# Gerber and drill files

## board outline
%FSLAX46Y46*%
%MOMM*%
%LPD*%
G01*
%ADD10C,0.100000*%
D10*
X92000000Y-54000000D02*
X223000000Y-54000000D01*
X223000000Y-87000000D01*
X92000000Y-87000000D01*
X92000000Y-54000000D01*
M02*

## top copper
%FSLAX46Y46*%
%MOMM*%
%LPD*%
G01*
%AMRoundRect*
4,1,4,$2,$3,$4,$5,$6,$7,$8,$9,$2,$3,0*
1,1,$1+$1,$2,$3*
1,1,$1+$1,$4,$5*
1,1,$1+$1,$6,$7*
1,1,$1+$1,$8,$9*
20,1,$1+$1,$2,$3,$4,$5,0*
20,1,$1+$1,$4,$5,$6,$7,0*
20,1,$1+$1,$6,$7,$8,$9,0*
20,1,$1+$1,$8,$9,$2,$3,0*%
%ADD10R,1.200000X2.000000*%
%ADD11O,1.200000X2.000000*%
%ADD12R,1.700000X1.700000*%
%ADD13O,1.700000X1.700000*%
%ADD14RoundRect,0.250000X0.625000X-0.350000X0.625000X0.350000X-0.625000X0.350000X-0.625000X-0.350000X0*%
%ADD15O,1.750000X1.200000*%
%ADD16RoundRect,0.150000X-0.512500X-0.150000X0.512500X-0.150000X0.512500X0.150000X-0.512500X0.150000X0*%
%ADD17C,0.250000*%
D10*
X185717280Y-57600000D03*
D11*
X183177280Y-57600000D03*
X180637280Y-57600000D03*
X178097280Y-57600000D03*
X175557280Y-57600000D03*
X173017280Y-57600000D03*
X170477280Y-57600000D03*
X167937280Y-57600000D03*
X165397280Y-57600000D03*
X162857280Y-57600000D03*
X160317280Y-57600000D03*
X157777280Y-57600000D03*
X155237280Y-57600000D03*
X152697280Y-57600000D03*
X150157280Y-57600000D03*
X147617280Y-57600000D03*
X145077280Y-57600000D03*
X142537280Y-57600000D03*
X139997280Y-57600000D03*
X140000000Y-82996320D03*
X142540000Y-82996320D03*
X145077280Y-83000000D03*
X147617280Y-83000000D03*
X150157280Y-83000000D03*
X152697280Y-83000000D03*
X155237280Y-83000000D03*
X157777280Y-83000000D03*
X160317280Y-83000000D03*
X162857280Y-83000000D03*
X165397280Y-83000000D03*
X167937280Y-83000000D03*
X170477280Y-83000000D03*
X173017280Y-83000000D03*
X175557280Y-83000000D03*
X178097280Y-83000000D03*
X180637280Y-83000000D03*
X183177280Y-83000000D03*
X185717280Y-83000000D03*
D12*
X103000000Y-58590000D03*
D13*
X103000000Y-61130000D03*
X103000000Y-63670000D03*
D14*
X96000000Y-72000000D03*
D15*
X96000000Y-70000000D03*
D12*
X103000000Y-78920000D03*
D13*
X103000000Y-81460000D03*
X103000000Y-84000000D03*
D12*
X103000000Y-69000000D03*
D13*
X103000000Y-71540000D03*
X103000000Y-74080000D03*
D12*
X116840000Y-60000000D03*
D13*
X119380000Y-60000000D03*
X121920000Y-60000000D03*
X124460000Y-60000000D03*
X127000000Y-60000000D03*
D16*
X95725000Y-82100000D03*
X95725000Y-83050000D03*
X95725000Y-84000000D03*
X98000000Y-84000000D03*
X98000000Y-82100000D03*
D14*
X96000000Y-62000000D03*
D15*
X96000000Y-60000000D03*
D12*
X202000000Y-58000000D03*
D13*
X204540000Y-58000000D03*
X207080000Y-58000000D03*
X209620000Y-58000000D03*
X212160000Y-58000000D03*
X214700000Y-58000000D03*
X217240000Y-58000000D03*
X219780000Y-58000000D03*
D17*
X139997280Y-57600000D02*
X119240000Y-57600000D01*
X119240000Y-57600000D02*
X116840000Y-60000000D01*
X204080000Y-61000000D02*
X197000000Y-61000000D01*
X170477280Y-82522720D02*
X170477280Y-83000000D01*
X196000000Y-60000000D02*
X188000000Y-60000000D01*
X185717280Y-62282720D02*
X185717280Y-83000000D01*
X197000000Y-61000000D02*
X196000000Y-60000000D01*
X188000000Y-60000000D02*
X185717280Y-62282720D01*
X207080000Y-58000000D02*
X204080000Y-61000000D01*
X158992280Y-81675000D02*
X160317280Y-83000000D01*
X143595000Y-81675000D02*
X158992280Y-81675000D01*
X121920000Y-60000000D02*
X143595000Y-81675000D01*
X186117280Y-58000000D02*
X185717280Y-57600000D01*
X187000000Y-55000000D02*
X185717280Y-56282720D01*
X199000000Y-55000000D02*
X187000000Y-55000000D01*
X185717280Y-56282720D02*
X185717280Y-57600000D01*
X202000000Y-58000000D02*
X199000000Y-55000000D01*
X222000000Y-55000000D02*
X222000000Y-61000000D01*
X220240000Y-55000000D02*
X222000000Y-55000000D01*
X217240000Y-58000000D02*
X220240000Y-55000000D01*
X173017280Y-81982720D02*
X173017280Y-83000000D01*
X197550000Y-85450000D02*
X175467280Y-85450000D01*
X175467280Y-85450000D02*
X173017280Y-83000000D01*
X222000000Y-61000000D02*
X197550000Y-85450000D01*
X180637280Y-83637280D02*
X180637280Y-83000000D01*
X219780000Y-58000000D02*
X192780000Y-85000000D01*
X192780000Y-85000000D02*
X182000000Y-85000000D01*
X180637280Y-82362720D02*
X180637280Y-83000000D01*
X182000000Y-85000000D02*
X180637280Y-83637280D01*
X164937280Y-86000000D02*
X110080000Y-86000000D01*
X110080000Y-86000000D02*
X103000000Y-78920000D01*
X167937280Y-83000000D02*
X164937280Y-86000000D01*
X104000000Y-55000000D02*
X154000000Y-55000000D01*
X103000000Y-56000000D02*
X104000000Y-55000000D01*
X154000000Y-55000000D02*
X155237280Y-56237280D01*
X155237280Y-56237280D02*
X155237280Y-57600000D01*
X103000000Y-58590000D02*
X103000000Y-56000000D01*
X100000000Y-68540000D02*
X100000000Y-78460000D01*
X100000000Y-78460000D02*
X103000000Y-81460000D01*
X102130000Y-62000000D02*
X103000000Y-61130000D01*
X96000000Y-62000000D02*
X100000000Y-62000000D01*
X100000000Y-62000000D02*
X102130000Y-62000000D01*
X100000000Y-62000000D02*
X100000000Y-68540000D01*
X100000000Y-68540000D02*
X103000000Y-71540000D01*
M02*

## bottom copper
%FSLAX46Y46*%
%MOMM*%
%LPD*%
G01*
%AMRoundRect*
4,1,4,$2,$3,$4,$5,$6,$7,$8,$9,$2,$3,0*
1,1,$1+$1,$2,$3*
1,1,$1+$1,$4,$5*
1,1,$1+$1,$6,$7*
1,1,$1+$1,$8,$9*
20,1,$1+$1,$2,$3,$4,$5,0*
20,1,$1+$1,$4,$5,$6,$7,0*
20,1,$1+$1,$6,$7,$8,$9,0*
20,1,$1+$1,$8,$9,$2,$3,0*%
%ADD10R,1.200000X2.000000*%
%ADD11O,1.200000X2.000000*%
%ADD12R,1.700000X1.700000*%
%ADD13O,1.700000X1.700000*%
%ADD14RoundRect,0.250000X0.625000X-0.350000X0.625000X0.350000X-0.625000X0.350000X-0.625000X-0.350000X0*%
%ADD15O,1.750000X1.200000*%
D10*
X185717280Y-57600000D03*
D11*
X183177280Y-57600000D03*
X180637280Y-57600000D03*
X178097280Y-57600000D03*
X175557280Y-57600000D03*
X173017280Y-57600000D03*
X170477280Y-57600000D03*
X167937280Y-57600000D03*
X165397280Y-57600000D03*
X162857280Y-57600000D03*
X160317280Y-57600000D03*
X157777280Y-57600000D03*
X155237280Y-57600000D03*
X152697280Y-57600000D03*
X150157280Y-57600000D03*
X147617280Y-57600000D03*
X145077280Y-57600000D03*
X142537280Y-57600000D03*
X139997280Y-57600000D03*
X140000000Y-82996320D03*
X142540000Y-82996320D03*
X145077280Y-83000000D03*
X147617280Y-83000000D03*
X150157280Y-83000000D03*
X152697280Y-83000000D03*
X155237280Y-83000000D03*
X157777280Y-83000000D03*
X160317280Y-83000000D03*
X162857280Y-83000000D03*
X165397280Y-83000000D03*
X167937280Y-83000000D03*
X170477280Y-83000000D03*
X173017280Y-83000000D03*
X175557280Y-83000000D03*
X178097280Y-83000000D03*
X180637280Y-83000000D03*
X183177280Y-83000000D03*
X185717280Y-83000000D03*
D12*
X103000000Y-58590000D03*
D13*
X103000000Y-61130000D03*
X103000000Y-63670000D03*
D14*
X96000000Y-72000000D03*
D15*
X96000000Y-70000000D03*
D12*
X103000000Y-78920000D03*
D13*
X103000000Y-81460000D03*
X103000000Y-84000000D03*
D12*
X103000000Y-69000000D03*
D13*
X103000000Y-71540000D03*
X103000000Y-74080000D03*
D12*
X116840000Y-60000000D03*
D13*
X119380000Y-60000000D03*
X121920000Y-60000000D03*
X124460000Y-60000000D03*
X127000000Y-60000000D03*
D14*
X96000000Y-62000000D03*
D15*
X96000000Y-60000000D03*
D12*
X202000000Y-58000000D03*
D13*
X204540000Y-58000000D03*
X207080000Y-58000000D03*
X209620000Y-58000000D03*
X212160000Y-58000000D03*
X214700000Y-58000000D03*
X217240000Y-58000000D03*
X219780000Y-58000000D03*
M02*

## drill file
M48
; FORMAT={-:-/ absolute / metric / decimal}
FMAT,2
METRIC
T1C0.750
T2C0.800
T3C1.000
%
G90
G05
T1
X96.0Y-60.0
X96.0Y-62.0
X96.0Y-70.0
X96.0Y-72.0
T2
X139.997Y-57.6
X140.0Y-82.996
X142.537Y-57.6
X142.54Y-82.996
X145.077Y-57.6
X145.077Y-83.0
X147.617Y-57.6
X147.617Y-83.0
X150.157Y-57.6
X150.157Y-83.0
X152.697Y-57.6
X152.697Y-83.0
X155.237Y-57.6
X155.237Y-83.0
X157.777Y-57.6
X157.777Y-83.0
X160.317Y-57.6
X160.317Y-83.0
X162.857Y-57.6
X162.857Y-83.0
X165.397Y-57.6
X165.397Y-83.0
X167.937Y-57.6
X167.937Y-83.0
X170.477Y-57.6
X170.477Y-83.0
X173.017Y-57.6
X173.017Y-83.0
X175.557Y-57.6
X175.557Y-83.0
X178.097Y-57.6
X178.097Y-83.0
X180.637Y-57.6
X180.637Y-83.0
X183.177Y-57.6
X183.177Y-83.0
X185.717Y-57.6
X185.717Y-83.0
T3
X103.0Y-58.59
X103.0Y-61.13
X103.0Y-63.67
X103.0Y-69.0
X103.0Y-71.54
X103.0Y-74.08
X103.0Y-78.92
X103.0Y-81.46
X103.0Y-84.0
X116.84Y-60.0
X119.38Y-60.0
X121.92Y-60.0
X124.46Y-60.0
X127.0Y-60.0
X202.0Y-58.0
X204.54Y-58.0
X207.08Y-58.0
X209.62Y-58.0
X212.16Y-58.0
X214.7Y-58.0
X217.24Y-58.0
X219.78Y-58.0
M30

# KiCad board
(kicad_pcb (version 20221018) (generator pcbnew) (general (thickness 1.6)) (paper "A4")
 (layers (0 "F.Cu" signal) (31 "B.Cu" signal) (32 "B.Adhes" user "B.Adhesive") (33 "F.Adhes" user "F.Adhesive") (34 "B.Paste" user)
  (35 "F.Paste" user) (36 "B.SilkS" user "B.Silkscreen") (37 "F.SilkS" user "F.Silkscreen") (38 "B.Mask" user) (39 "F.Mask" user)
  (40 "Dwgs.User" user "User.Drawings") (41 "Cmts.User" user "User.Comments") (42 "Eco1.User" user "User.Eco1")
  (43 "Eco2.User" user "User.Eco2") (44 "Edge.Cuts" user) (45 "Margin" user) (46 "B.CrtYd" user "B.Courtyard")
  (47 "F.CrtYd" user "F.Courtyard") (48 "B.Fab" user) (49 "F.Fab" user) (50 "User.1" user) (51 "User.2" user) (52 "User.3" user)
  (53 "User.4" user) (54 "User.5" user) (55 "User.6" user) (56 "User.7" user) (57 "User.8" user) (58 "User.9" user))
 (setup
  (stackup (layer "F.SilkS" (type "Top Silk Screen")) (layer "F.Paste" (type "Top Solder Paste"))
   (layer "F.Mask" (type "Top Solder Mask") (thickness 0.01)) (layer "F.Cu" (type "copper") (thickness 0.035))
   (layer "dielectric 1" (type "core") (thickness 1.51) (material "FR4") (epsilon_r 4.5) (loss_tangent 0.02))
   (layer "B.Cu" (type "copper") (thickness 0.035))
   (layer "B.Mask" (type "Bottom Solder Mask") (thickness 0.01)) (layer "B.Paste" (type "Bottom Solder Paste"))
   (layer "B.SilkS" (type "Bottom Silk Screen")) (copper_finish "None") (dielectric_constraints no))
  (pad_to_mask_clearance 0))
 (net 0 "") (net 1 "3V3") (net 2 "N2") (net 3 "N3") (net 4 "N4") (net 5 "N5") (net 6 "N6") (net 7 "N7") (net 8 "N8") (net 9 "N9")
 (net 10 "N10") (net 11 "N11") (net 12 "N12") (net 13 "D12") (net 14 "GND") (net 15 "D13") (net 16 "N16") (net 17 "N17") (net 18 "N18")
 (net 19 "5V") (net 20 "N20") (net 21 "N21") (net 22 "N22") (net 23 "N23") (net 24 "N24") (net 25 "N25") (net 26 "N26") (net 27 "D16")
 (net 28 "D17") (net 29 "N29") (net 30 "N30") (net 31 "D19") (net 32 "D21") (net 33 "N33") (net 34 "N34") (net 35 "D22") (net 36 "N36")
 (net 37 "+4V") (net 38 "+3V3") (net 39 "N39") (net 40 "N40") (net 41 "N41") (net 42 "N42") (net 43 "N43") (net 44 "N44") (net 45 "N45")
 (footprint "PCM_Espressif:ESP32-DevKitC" (layer "F.Cu") (at 185.71728 57.6 -90)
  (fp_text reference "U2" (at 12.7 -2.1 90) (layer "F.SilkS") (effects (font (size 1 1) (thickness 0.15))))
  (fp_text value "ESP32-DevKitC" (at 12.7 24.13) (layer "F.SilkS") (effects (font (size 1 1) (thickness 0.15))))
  (pad "1" thru_hole rect (at 0 0 180) (size 1.2 2) (drill 0.8) (layers "*.Cu" "*.Mask") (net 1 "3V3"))
  (pad "2" thru_hole oval (at 0 2.54 180) (size 1.2 2) (drill 0.8) (layers "*.Cu" "*.Mask") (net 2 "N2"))
  (pad "3" thru_hole oval (at 0 5.08 180) (size 1.2 2) (drill 0.8) (layers "*.Cu" "*.Mask") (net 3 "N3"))
  (pad "4" thru_hole oval (at 0 7.62 180) (size 1.2 2) (drill 0.8) (layers "*.Cu" "*.Mask") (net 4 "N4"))
  (pad "5" thru_hole oval (at 0 10.16 180) (size 1.2 2) (drill 0.8) (layers "*.Cu" "*.Mask") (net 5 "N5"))
  (pad "6" thru_hole oval (at 0 12.7 180) (size 1.2 2) (drill 0.8) (layers "*.Cu" "*.Mask") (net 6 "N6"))
  (pad "7" thru_hole oval (at 0 15.24 180) (size 1.2 2) (drill 0.8) (layers "*.Cu" "*.Mask") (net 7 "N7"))
  (pad "8" thru_hole oval (at 0 17.78 180) (size 1.2 2) (drill 0.8) (layers "*.Cu" "*.Mask") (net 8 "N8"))
  (pad "9" thru_hole oval (at 0 20.32 180) (size 1.2 2) (drill 0.8) (layers "*.Cu" "*.Mask") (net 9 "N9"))
  (pad "10" thru_hole oval (at 0 22.86 180) (size 1.2 2) (drill 0.8) (layers "*.Cu" "*.Mask") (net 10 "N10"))
  (pad "11" thru_hole oval (at 0 25.4 180) (size 1.2 2) (drill 0.8) (layers "*.Cu" "*.Mask") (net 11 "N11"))
  (pad "12" thru_hole oval (at 0 27.94 180) (size 1.2 2) (drill 0.8) (layers "*.Cu" "*.Mask") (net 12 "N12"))
  (pad "13" thru_hole oval (at 0 30.48 180) (size 1.2 2) (drill 0.8) (layers "*.Cu" "*.Mask") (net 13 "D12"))
  (pad "14" thru_hole oval (at 0 33.02 180) (size 1.2 2) (drill 0.8) (layers "*.Cu" "*.Mask") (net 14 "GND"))
  (pad "15" thru_hole oval (at 0 35.56 180) (size 1.2 2) (drill 0.8) (layers "*.Cu" "*.Mask") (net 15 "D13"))
  (pad "16" thru_hole oval (at 0 38.1 180) (size 1.2 2) (drill 0.8) (layers "*.Cu" "*.Mask") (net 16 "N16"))
  (pad "17" thru_hole oval (at 0 40.64 180) (size 1.2 2) (drill 0.8) (layers "*.Cu" "*.Mask") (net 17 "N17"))
  (pad "18" thru_hole oval (at 0 43.18 180) (size 1.2 2) (drill 0.8) (layers "*.Cu" "*.Mask") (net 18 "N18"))
  (pad "19" thru_hole oval (at 0 45.72 180) (size 1.2 2) (drill 0.8) (layers "*.Cu" "*.Mask") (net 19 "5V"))
  (pad "20" thru_hole oval (at 25.39632 45.71728 180) (size 1.2 2) (drill 0.8) (layers "*.Cu" "*.Mask") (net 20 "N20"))
  (pad "21" thru_hole oval (at 25.39632 43.17728 180) (size 1.2 2) (drill 0.8) (layers "*.Cu" "*.Mask") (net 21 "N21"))
  (pad "22" thru_hole oval (at 25.4 40.64 180) (size 1.2 2) (drill 0.8) (layers "*.Cu" "*.Mask") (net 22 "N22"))
  (pad "23" thru_hole oval (at 25.4 38.1 180) (size 1.2 2) (drill 0.8) (layers "*.Cu" "*.Mask") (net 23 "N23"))
  (pad "24" thru_hole oval (at 25.4 35.56 180) (size 1.2 2) (drill 0.8) (layers "*.Cu" "*.Mask") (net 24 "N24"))
  (pad "25" thru_hole oval (at 25.4 33.02 180) (size 1.2 2) (drill 0.8) (layers "*.Cu" "*.Mask") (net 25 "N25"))
  (pad "26" thru_hole oval (at 25.4 30.48 180) (size 1.2 2) (drill 0.8) (layers "*.Cu" "*.Mask") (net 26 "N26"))
  (pad "27" thru_hole oval (at 25.4 27.94 180) (size 1.2 2) (drill 0.8) (layers "*.Cu" "*.Mask") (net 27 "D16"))
  (pad "28" thru_hole oval (at 25.4 25.4 180) (size 1.2 2) (drill 0.8) (layers "*.Cu" "*.Mask") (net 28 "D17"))
  (pad "29" thru_hole oval (at 25.4 22.86 180) (size 1.2 2) (drill 0.8) (layers "*.Cu" "*.Mask") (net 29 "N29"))
  (pad "30" thru_hole oval (at 25.4 20.32 180) (size 1.2 2) (drill 0.8) (layers "*.Cu" "*.Mask") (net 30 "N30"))
  (pad "31" thru_hole oval (at 25.4 17.78 180) (size 1.2 2) (drill 0.8) (layers "*.Cu" "*.Mask") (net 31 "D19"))
  (pad "32" thru_hole oval (at 25.4 15.24 180) (size 1.2 2) (drill 0.8) (layers "*.Cu" "*.Mask") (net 14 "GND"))
  (pad "33" thru_hole oval (at 25.4 12.7 180) (size 1.2 2) (drill 0.8) (layers "*.Cu" "*.Mask") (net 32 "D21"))
  (pad "34" thru_hole oval (at 25.4 10.16 180) (size 1.2 2) (drill 0.8) (layers "*.Cu" "*.Mask") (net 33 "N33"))
  (pad "35" thru_hole oval (at 25.4 7.62 180) (size 1.2 2) (drill 0.8) (layers "*.Cu" "*.Mask") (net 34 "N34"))
  (pad "36" thru_hole oval (at 25.4 5.08 180) (size 1.2 2) (drill 0.8) (layers "*.Cu" "*.Mask") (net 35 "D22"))
  (pad "37" thru_hole oval (at 25.4 2.54 180) (size 1.2 2) (drill 0.8) (layers "*.Cu" "*.Mask") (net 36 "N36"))
  (pad "38" thru_hole oval (at 25.4 0 180) (size 1.2 2) (drill 0.8) (layers "*.Cu" "*.Mask") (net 14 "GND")))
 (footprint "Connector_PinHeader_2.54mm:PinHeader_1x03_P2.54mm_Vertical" (layer "F.Cu") (at 103 58.59)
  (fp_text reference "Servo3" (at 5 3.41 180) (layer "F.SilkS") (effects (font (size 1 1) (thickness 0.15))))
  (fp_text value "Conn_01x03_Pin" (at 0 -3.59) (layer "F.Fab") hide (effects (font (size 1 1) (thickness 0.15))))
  (pad "1" thru_hole rect (at 0 0) (size 1.7 1.7) (drill 1) (layers "*.Cu" "*.Mask") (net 13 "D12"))
  (pad "2" thru_hole oval (at 0 2.54) (size 1.7 1.7) (drill 1) (layers "*.Cu" "*.Mask") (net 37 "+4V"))
  (pad "3" thru_hole oval (at 0 5.08) (size 1.7 1.7) (drill 1) (layers "*.Cu" "*.Mask") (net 14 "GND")))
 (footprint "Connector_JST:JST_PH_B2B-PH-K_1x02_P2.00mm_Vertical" (layer "F.Cu") (at 96 72 90)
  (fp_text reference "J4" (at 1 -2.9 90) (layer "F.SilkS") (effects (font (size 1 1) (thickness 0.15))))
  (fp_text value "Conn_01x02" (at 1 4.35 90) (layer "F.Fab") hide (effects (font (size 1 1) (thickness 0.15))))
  (pad "1" thru_hole roundrect (at 0 0 90) (size 1.2 1.75) (drill 0.75) (layers "*.Cu" "*.Mask") (roundrect_rratio 0.208333) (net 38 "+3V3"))
  (pad "2" thru_hole oval (at 2 0 90) (size 1.2 1.75) (drill 0.75) (layers "*.Cu" "*.Mask") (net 14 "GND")))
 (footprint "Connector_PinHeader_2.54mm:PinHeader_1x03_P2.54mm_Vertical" (layer "F.Cu") (at 103 78.92)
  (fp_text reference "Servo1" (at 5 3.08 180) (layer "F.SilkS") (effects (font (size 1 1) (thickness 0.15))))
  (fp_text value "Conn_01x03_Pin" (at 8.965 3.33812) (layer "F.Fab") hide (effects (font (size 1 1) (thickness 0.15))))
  (pad "1" thru_hole rect (at 0 0) (size 1.7 1.7) (drill 1) (layers "*.Cu" "*.Mask") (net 31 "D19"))
  (pad "2" thru_hole oval (at 0 2.54) (size 1.7 1.7) (drill 1) (layers "*.Cu" "*.Mask") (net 37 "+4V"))
  (pad "3" thru_hole oval (at 0 5.08) (size 1.7 1.7) (drill 1) (layers "*.Cu" "*.Mask") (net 14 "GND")))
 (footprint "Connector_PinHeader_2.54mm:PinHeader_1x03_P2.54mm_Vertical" (layer "F.Cu") (at 103 69)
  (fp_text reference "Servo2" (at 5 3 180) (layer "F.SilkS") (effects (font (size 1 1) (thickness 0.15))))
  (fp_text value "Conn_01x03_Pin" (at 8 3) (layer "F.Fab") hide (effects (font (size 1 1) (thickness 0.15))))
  (pad "1" thru_hole rect (at 0 0) (size 1.7 1.7) (drill 1) (layers "*.Cu" "*.Mask") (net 15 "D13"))
  (pad "2" thru_hole oval (at 0 2.54) (size 1.7 1.7) (drill 1) (layers "*.Cu" "*.Mask") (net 37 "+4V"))
  (pad "3" thru_hole oval (at 0 5.08) (size 1.7 1.7) (drill 1) (layers "*.Cu" "*.Mask") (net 14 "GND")))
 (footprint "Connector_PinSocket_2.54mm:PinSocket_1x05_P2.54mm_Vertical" (layer "F.Cu") (at 116.84 60 90)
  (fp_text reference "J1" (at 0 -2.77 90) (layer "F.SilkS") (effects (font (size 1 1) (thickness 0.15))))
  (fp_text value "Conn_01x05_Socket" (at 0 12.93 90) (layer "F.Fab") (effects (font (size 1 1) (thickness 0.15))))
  (pad "1" thru_hole rect (at 0 0 90) (size 1.7 1.7) (drill 1) (layers "*.Cu" "*.Mask") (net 19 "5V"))
  (pad "2" thru_hole oval (at 0 2.54 90) (size 1.7 1.7) (drill 1) (layers "*.Cu" "*.Mask") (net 14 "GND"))
  (pad "3" thru_hole oval (at 0 5.08 90) (size 1.7 1.7) (drill 1) (layers "*.Cu" "*.Mask") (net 28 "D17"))
  (pad "4" thru_hole oval (at 0 7.62 90) (size 1.7 1.7) (drill 1) (layers "*.Cu" "*.Mask") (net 27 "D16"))
  (pad "5" thru_hole oval (at 0 10.16 90) (size 1.7 1.7) (drill 1) (layers "*.Cu" "*.Mask") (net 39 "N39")))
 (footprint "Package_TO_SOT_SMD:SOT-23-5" (layer "F.Cu") (at 96.8625 83.05)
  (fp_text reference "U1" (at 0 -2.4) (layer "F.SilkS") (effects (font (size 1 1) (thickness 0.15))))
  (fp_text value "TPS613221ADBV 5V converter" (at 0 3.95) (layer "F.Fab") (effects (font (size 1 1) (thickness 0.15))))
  (pad "1" smd roundrect (at -1.1375 -0.95) (size 1.325 0.6) (layers "F.Cu" "F.Paste" "F.Mask") (roundrect_rratio 0.25) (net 38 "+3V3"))
  (pad "2" smd roundrect (at -1.1375 0) (size 1.325 0.6) (layers "F.Cu" "F.Paste" "F.Mask") (roundrect_rratio 0.25) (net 14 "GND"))
  (pad "3" smd roundrect (at -1.1375 0.95) (size 1.325 0.6) (layers "F.Cu" "F.Paste" "F.Mask") (roundrect_rratio 0.25) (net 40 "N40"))
  (pad "4" smd roundrect (at 1.1375 0.95) (size 1.325 0.6) (layers "F.Cu" "F.Paste" "F.Mask") (roundrect_rratio 0.25) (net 19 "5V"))
  (pad "5" smd roundrect (at 1.1375 -0.95) (size 1.325 0.6) (layers "F.Cu" "F.Paste" "F.Mask") (roundrect_rratio 0.25) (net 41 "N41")))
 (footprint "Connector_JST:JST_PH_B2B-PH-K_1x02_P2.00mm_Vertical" (layer "F.Cu") (at 96 62 90)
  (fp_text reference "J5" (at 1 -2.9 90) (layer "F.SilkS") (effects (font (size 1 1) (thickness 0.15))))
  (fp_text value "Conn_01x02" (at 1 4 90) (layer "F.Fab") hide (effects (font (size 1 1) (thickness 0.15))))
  (pad "1" thru_hole roundrect (at 0 0 90) (size 1.2 1.75) (drill 0.75) (layers "*.Cu" "*.Mask") (roundrect_rratio 0.208333) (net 37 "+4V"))
  (pad "2" thru_hole oval (at 2 0 90) (size 1.2 1.75) (drill 0.75) (layers "*.Cu" "*.Mask") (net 14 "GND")))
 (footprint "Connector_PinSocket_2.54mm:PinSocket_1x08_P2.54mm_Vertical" (layer "F.Cu") (at 202 58 90)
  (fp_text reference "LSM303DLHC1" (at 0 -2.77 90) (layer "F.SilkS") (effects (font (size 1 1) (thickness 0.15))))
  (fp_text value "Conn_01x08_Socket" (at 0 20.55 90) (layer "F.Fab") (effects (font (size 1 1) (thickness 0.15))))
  (pad "1" thru_hole rect (at 0 0 90) (size 1.7 1.7) (drill 1) (layers "*.Cu" "*.Mask") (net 1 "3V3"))
  (pad "2" thru_hole oval (at 0 2.54 90) (size 1.7 1.7) (drill 1) (layers "*.Cu" "*.Mask") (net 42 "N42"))
  (pad "3" thru_hole oval (at 0 5.08 90) (size 1.7 1.7) (drill 1) (layers "*.Cu" "*.Mask") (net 14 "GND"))
  (pad "4" thru_hole oval (at 0 7.62 90) (size 1.7 1.7) (drill 1) (layers "*.Cu" "*.Mask") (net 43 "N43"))
  (pad "5" thru_hole oval (at 0 10.16 90) (size 1.7 1.7) (drill 1) (layers "*.Cu" "*.Mask") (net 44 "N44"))
  (pad "6" thru_hole oval (at 0 12.7 90) (size 1.7 1.7) (drill 1) (layers "*.Cu" "*.Mask") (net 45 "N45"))
  (pad "7" thru_hole oval (at 0 15.24 90) (size 1.7 1.7) (drill 1) (layers "*.Cu" "*.Mask") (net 32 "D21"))
  (pad "8" thru_hole oval (at 0 17.78 90) (size 1.7 1.7) (drill 1) (layers "*.Cu" "*.Mask") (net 35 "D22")))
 (gr_rect (start 92 54) (end 223 87) (stroke (width 0.1) (type default)) (fill none) (layer "Edge.Cuts"))
 (segment (start 139.99728 57.6) (end 119.24 57.6) (width 0.25) (layer "F.Cu") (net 19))
 (segment (start 119.24 57.6) (end 116.84 60) (width 0.25) (layer "F.Cu") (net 19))
 (segment (start 204.08 61) (end 197 61) (width 0.25) (layer "F.Cu") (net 14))
 (segment (start 170.47728 82.52272) (end 170.47728 83) (width 0.25) (layer "F.Cu") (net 14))
 (segment (start 196 60) (end 188 60) (width 0.25) (layer "F.Cu") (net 14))
 (segment (start 185.71728 62.28272) (end 185.71728 83) (width 0.25) (layer "F.Cu") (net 14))
 (segment (start 197 61) (end 196 60) (width 0.25) (layer "F.Cu") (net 14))
 (segment (start 188 60) (end 185.71728 62.28272) (width 0.25) (layer "F.Cu") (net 14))
 (segment (start 207.08 58) (end 204.08 61) (width 0.25) (layer "F.Cu") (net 14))
 (segment (start 158.99228 81.675) (end 160.31728 83) (width 0.25) (layer "F.Cu") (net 28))
 (segment (start 143.595 81.675) (end 158.99228 81.675) (width 0.25) (layer "F.Cu") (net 28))
 (segment (start 121.92 60) (end 143.595 81.675) (width 0.25) (layer "F.Cu") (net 28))
 (segment (start 186.11728 58) (end 185.71728 57.6) (width 0.25) (layer "F.Cu") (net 1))
 (segment (start 187 55) (end 185.71728 56.28272) (width 0.25) (layer "F.Cu") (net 1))
 (segment (start 199 55) (end 187 55) (width 0.25) (layer "F.Cu") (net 1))
 (segment (start 185.71728 56.28272) (end 185.71728 57.6) (width 0.25) (layer "F.Cu") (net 1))
 (segment (start 202 58) (end 199 55) (width 0.25) (layer "F.Cu") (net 1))
 (segment (start 222 55) (end 222 61) (width 0.25) (layer "F.Cu") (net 32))
 (segment (start 220.24 55) (end 222 55) (width 0.25) (layer "F.Cu") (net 32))
 (segment (start 217.24 58) (end 220.24 55) (width 0.25) (layer "F.Cu") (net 32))
 (segment (start 173.01728 81.98272) (end 173.01728 83) (width 0.25) (layer "F.Cu") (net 32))
 (segment (start 197.55 85.45) (end 175.46728 85.45) (width 0.25) (layer "F.Cu") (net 32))
 (segment (start 175.46728 85.45) (end 173.01728 83) (width 0.25) (layer "F.Cu") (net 32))
 (segment (start 222 61) (end 197.55 85.45) (width 0.25) (layer "F.Cu") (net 32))
 (segment (start 180.63728 83.63728) (end 180.63728 83) (width 0.25) (layer "F.Cu") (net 35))
 (segment (start 219.78 58) (end 192.78 85) (width 0.25) (layer "F.Cu") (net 35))
 (segment (start 192.78 85) (end 182 85) (width 0.25) (layer "F.Cu") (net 35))
 (segment (start 180.63728 82.36272) (end 180.63728 83) (width 0.25) (layer "F.Cu") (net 35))
 (segment (start 182 85) (end 180.63728 83.63728) (width 0.25) (layer "F.Cu") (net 35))
 (segment (start 164.93728 86) (end 110.08 86) (width 0.25) (layer "F.Cu") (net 31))
 (segment (start 110.08 86) (end 103 78.92) (width 0.25) (layer "F.Cu") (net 31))
 (segment (start 167.93728 83) (end 164.93728 86) (width 0.25) (layer "F.Cu") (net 31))
 (segment (start 104 55) (end 154 55) (width 0.25) (layer "F.Cu") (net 13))
 (segment (start 103 56) (end 104 55) (width 0.25) (layer "F.Cu") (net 13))
 (segment (start 154 55) (end 155.23728 56.23728) (width 0.25) (layer "F.Cu") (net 13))
 (segment (start 155.23728 56.23728) (end 155.23728 57.6) (width 0.25) (layer "F.Cu") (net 13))
 (segment (start 103 58.59) (end 103 56) (width 0.25) (layer "F.Cu") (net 13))
 (segment (start 100 68.54) (end 100 78.46) (width 0.25) (layer "F.Cu") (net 37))
 (segment (start 100 78.46) (end 103 81.46) (width 0.25) (layer "F.Cu") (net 37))
 (segment (start 102.13 62) (end 103 61.13) (width 0.25) (layer "F.Cu") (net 37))
 (segment (start 96 62) (end 100 62) (width 0.25) (layer "F.Cu") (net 37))
 (segment (start 100 62) (end 102.13 62) (width 0.25) (layer "F.Cu") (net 37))
 (segment (start 100 62) (end 100 68.54) (width 0.25) (layer "F.Cu") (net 37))
 (segment (start 100 68.54) (end 103 71.54) (width 0.25) (layer "F.Cu") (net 37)))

